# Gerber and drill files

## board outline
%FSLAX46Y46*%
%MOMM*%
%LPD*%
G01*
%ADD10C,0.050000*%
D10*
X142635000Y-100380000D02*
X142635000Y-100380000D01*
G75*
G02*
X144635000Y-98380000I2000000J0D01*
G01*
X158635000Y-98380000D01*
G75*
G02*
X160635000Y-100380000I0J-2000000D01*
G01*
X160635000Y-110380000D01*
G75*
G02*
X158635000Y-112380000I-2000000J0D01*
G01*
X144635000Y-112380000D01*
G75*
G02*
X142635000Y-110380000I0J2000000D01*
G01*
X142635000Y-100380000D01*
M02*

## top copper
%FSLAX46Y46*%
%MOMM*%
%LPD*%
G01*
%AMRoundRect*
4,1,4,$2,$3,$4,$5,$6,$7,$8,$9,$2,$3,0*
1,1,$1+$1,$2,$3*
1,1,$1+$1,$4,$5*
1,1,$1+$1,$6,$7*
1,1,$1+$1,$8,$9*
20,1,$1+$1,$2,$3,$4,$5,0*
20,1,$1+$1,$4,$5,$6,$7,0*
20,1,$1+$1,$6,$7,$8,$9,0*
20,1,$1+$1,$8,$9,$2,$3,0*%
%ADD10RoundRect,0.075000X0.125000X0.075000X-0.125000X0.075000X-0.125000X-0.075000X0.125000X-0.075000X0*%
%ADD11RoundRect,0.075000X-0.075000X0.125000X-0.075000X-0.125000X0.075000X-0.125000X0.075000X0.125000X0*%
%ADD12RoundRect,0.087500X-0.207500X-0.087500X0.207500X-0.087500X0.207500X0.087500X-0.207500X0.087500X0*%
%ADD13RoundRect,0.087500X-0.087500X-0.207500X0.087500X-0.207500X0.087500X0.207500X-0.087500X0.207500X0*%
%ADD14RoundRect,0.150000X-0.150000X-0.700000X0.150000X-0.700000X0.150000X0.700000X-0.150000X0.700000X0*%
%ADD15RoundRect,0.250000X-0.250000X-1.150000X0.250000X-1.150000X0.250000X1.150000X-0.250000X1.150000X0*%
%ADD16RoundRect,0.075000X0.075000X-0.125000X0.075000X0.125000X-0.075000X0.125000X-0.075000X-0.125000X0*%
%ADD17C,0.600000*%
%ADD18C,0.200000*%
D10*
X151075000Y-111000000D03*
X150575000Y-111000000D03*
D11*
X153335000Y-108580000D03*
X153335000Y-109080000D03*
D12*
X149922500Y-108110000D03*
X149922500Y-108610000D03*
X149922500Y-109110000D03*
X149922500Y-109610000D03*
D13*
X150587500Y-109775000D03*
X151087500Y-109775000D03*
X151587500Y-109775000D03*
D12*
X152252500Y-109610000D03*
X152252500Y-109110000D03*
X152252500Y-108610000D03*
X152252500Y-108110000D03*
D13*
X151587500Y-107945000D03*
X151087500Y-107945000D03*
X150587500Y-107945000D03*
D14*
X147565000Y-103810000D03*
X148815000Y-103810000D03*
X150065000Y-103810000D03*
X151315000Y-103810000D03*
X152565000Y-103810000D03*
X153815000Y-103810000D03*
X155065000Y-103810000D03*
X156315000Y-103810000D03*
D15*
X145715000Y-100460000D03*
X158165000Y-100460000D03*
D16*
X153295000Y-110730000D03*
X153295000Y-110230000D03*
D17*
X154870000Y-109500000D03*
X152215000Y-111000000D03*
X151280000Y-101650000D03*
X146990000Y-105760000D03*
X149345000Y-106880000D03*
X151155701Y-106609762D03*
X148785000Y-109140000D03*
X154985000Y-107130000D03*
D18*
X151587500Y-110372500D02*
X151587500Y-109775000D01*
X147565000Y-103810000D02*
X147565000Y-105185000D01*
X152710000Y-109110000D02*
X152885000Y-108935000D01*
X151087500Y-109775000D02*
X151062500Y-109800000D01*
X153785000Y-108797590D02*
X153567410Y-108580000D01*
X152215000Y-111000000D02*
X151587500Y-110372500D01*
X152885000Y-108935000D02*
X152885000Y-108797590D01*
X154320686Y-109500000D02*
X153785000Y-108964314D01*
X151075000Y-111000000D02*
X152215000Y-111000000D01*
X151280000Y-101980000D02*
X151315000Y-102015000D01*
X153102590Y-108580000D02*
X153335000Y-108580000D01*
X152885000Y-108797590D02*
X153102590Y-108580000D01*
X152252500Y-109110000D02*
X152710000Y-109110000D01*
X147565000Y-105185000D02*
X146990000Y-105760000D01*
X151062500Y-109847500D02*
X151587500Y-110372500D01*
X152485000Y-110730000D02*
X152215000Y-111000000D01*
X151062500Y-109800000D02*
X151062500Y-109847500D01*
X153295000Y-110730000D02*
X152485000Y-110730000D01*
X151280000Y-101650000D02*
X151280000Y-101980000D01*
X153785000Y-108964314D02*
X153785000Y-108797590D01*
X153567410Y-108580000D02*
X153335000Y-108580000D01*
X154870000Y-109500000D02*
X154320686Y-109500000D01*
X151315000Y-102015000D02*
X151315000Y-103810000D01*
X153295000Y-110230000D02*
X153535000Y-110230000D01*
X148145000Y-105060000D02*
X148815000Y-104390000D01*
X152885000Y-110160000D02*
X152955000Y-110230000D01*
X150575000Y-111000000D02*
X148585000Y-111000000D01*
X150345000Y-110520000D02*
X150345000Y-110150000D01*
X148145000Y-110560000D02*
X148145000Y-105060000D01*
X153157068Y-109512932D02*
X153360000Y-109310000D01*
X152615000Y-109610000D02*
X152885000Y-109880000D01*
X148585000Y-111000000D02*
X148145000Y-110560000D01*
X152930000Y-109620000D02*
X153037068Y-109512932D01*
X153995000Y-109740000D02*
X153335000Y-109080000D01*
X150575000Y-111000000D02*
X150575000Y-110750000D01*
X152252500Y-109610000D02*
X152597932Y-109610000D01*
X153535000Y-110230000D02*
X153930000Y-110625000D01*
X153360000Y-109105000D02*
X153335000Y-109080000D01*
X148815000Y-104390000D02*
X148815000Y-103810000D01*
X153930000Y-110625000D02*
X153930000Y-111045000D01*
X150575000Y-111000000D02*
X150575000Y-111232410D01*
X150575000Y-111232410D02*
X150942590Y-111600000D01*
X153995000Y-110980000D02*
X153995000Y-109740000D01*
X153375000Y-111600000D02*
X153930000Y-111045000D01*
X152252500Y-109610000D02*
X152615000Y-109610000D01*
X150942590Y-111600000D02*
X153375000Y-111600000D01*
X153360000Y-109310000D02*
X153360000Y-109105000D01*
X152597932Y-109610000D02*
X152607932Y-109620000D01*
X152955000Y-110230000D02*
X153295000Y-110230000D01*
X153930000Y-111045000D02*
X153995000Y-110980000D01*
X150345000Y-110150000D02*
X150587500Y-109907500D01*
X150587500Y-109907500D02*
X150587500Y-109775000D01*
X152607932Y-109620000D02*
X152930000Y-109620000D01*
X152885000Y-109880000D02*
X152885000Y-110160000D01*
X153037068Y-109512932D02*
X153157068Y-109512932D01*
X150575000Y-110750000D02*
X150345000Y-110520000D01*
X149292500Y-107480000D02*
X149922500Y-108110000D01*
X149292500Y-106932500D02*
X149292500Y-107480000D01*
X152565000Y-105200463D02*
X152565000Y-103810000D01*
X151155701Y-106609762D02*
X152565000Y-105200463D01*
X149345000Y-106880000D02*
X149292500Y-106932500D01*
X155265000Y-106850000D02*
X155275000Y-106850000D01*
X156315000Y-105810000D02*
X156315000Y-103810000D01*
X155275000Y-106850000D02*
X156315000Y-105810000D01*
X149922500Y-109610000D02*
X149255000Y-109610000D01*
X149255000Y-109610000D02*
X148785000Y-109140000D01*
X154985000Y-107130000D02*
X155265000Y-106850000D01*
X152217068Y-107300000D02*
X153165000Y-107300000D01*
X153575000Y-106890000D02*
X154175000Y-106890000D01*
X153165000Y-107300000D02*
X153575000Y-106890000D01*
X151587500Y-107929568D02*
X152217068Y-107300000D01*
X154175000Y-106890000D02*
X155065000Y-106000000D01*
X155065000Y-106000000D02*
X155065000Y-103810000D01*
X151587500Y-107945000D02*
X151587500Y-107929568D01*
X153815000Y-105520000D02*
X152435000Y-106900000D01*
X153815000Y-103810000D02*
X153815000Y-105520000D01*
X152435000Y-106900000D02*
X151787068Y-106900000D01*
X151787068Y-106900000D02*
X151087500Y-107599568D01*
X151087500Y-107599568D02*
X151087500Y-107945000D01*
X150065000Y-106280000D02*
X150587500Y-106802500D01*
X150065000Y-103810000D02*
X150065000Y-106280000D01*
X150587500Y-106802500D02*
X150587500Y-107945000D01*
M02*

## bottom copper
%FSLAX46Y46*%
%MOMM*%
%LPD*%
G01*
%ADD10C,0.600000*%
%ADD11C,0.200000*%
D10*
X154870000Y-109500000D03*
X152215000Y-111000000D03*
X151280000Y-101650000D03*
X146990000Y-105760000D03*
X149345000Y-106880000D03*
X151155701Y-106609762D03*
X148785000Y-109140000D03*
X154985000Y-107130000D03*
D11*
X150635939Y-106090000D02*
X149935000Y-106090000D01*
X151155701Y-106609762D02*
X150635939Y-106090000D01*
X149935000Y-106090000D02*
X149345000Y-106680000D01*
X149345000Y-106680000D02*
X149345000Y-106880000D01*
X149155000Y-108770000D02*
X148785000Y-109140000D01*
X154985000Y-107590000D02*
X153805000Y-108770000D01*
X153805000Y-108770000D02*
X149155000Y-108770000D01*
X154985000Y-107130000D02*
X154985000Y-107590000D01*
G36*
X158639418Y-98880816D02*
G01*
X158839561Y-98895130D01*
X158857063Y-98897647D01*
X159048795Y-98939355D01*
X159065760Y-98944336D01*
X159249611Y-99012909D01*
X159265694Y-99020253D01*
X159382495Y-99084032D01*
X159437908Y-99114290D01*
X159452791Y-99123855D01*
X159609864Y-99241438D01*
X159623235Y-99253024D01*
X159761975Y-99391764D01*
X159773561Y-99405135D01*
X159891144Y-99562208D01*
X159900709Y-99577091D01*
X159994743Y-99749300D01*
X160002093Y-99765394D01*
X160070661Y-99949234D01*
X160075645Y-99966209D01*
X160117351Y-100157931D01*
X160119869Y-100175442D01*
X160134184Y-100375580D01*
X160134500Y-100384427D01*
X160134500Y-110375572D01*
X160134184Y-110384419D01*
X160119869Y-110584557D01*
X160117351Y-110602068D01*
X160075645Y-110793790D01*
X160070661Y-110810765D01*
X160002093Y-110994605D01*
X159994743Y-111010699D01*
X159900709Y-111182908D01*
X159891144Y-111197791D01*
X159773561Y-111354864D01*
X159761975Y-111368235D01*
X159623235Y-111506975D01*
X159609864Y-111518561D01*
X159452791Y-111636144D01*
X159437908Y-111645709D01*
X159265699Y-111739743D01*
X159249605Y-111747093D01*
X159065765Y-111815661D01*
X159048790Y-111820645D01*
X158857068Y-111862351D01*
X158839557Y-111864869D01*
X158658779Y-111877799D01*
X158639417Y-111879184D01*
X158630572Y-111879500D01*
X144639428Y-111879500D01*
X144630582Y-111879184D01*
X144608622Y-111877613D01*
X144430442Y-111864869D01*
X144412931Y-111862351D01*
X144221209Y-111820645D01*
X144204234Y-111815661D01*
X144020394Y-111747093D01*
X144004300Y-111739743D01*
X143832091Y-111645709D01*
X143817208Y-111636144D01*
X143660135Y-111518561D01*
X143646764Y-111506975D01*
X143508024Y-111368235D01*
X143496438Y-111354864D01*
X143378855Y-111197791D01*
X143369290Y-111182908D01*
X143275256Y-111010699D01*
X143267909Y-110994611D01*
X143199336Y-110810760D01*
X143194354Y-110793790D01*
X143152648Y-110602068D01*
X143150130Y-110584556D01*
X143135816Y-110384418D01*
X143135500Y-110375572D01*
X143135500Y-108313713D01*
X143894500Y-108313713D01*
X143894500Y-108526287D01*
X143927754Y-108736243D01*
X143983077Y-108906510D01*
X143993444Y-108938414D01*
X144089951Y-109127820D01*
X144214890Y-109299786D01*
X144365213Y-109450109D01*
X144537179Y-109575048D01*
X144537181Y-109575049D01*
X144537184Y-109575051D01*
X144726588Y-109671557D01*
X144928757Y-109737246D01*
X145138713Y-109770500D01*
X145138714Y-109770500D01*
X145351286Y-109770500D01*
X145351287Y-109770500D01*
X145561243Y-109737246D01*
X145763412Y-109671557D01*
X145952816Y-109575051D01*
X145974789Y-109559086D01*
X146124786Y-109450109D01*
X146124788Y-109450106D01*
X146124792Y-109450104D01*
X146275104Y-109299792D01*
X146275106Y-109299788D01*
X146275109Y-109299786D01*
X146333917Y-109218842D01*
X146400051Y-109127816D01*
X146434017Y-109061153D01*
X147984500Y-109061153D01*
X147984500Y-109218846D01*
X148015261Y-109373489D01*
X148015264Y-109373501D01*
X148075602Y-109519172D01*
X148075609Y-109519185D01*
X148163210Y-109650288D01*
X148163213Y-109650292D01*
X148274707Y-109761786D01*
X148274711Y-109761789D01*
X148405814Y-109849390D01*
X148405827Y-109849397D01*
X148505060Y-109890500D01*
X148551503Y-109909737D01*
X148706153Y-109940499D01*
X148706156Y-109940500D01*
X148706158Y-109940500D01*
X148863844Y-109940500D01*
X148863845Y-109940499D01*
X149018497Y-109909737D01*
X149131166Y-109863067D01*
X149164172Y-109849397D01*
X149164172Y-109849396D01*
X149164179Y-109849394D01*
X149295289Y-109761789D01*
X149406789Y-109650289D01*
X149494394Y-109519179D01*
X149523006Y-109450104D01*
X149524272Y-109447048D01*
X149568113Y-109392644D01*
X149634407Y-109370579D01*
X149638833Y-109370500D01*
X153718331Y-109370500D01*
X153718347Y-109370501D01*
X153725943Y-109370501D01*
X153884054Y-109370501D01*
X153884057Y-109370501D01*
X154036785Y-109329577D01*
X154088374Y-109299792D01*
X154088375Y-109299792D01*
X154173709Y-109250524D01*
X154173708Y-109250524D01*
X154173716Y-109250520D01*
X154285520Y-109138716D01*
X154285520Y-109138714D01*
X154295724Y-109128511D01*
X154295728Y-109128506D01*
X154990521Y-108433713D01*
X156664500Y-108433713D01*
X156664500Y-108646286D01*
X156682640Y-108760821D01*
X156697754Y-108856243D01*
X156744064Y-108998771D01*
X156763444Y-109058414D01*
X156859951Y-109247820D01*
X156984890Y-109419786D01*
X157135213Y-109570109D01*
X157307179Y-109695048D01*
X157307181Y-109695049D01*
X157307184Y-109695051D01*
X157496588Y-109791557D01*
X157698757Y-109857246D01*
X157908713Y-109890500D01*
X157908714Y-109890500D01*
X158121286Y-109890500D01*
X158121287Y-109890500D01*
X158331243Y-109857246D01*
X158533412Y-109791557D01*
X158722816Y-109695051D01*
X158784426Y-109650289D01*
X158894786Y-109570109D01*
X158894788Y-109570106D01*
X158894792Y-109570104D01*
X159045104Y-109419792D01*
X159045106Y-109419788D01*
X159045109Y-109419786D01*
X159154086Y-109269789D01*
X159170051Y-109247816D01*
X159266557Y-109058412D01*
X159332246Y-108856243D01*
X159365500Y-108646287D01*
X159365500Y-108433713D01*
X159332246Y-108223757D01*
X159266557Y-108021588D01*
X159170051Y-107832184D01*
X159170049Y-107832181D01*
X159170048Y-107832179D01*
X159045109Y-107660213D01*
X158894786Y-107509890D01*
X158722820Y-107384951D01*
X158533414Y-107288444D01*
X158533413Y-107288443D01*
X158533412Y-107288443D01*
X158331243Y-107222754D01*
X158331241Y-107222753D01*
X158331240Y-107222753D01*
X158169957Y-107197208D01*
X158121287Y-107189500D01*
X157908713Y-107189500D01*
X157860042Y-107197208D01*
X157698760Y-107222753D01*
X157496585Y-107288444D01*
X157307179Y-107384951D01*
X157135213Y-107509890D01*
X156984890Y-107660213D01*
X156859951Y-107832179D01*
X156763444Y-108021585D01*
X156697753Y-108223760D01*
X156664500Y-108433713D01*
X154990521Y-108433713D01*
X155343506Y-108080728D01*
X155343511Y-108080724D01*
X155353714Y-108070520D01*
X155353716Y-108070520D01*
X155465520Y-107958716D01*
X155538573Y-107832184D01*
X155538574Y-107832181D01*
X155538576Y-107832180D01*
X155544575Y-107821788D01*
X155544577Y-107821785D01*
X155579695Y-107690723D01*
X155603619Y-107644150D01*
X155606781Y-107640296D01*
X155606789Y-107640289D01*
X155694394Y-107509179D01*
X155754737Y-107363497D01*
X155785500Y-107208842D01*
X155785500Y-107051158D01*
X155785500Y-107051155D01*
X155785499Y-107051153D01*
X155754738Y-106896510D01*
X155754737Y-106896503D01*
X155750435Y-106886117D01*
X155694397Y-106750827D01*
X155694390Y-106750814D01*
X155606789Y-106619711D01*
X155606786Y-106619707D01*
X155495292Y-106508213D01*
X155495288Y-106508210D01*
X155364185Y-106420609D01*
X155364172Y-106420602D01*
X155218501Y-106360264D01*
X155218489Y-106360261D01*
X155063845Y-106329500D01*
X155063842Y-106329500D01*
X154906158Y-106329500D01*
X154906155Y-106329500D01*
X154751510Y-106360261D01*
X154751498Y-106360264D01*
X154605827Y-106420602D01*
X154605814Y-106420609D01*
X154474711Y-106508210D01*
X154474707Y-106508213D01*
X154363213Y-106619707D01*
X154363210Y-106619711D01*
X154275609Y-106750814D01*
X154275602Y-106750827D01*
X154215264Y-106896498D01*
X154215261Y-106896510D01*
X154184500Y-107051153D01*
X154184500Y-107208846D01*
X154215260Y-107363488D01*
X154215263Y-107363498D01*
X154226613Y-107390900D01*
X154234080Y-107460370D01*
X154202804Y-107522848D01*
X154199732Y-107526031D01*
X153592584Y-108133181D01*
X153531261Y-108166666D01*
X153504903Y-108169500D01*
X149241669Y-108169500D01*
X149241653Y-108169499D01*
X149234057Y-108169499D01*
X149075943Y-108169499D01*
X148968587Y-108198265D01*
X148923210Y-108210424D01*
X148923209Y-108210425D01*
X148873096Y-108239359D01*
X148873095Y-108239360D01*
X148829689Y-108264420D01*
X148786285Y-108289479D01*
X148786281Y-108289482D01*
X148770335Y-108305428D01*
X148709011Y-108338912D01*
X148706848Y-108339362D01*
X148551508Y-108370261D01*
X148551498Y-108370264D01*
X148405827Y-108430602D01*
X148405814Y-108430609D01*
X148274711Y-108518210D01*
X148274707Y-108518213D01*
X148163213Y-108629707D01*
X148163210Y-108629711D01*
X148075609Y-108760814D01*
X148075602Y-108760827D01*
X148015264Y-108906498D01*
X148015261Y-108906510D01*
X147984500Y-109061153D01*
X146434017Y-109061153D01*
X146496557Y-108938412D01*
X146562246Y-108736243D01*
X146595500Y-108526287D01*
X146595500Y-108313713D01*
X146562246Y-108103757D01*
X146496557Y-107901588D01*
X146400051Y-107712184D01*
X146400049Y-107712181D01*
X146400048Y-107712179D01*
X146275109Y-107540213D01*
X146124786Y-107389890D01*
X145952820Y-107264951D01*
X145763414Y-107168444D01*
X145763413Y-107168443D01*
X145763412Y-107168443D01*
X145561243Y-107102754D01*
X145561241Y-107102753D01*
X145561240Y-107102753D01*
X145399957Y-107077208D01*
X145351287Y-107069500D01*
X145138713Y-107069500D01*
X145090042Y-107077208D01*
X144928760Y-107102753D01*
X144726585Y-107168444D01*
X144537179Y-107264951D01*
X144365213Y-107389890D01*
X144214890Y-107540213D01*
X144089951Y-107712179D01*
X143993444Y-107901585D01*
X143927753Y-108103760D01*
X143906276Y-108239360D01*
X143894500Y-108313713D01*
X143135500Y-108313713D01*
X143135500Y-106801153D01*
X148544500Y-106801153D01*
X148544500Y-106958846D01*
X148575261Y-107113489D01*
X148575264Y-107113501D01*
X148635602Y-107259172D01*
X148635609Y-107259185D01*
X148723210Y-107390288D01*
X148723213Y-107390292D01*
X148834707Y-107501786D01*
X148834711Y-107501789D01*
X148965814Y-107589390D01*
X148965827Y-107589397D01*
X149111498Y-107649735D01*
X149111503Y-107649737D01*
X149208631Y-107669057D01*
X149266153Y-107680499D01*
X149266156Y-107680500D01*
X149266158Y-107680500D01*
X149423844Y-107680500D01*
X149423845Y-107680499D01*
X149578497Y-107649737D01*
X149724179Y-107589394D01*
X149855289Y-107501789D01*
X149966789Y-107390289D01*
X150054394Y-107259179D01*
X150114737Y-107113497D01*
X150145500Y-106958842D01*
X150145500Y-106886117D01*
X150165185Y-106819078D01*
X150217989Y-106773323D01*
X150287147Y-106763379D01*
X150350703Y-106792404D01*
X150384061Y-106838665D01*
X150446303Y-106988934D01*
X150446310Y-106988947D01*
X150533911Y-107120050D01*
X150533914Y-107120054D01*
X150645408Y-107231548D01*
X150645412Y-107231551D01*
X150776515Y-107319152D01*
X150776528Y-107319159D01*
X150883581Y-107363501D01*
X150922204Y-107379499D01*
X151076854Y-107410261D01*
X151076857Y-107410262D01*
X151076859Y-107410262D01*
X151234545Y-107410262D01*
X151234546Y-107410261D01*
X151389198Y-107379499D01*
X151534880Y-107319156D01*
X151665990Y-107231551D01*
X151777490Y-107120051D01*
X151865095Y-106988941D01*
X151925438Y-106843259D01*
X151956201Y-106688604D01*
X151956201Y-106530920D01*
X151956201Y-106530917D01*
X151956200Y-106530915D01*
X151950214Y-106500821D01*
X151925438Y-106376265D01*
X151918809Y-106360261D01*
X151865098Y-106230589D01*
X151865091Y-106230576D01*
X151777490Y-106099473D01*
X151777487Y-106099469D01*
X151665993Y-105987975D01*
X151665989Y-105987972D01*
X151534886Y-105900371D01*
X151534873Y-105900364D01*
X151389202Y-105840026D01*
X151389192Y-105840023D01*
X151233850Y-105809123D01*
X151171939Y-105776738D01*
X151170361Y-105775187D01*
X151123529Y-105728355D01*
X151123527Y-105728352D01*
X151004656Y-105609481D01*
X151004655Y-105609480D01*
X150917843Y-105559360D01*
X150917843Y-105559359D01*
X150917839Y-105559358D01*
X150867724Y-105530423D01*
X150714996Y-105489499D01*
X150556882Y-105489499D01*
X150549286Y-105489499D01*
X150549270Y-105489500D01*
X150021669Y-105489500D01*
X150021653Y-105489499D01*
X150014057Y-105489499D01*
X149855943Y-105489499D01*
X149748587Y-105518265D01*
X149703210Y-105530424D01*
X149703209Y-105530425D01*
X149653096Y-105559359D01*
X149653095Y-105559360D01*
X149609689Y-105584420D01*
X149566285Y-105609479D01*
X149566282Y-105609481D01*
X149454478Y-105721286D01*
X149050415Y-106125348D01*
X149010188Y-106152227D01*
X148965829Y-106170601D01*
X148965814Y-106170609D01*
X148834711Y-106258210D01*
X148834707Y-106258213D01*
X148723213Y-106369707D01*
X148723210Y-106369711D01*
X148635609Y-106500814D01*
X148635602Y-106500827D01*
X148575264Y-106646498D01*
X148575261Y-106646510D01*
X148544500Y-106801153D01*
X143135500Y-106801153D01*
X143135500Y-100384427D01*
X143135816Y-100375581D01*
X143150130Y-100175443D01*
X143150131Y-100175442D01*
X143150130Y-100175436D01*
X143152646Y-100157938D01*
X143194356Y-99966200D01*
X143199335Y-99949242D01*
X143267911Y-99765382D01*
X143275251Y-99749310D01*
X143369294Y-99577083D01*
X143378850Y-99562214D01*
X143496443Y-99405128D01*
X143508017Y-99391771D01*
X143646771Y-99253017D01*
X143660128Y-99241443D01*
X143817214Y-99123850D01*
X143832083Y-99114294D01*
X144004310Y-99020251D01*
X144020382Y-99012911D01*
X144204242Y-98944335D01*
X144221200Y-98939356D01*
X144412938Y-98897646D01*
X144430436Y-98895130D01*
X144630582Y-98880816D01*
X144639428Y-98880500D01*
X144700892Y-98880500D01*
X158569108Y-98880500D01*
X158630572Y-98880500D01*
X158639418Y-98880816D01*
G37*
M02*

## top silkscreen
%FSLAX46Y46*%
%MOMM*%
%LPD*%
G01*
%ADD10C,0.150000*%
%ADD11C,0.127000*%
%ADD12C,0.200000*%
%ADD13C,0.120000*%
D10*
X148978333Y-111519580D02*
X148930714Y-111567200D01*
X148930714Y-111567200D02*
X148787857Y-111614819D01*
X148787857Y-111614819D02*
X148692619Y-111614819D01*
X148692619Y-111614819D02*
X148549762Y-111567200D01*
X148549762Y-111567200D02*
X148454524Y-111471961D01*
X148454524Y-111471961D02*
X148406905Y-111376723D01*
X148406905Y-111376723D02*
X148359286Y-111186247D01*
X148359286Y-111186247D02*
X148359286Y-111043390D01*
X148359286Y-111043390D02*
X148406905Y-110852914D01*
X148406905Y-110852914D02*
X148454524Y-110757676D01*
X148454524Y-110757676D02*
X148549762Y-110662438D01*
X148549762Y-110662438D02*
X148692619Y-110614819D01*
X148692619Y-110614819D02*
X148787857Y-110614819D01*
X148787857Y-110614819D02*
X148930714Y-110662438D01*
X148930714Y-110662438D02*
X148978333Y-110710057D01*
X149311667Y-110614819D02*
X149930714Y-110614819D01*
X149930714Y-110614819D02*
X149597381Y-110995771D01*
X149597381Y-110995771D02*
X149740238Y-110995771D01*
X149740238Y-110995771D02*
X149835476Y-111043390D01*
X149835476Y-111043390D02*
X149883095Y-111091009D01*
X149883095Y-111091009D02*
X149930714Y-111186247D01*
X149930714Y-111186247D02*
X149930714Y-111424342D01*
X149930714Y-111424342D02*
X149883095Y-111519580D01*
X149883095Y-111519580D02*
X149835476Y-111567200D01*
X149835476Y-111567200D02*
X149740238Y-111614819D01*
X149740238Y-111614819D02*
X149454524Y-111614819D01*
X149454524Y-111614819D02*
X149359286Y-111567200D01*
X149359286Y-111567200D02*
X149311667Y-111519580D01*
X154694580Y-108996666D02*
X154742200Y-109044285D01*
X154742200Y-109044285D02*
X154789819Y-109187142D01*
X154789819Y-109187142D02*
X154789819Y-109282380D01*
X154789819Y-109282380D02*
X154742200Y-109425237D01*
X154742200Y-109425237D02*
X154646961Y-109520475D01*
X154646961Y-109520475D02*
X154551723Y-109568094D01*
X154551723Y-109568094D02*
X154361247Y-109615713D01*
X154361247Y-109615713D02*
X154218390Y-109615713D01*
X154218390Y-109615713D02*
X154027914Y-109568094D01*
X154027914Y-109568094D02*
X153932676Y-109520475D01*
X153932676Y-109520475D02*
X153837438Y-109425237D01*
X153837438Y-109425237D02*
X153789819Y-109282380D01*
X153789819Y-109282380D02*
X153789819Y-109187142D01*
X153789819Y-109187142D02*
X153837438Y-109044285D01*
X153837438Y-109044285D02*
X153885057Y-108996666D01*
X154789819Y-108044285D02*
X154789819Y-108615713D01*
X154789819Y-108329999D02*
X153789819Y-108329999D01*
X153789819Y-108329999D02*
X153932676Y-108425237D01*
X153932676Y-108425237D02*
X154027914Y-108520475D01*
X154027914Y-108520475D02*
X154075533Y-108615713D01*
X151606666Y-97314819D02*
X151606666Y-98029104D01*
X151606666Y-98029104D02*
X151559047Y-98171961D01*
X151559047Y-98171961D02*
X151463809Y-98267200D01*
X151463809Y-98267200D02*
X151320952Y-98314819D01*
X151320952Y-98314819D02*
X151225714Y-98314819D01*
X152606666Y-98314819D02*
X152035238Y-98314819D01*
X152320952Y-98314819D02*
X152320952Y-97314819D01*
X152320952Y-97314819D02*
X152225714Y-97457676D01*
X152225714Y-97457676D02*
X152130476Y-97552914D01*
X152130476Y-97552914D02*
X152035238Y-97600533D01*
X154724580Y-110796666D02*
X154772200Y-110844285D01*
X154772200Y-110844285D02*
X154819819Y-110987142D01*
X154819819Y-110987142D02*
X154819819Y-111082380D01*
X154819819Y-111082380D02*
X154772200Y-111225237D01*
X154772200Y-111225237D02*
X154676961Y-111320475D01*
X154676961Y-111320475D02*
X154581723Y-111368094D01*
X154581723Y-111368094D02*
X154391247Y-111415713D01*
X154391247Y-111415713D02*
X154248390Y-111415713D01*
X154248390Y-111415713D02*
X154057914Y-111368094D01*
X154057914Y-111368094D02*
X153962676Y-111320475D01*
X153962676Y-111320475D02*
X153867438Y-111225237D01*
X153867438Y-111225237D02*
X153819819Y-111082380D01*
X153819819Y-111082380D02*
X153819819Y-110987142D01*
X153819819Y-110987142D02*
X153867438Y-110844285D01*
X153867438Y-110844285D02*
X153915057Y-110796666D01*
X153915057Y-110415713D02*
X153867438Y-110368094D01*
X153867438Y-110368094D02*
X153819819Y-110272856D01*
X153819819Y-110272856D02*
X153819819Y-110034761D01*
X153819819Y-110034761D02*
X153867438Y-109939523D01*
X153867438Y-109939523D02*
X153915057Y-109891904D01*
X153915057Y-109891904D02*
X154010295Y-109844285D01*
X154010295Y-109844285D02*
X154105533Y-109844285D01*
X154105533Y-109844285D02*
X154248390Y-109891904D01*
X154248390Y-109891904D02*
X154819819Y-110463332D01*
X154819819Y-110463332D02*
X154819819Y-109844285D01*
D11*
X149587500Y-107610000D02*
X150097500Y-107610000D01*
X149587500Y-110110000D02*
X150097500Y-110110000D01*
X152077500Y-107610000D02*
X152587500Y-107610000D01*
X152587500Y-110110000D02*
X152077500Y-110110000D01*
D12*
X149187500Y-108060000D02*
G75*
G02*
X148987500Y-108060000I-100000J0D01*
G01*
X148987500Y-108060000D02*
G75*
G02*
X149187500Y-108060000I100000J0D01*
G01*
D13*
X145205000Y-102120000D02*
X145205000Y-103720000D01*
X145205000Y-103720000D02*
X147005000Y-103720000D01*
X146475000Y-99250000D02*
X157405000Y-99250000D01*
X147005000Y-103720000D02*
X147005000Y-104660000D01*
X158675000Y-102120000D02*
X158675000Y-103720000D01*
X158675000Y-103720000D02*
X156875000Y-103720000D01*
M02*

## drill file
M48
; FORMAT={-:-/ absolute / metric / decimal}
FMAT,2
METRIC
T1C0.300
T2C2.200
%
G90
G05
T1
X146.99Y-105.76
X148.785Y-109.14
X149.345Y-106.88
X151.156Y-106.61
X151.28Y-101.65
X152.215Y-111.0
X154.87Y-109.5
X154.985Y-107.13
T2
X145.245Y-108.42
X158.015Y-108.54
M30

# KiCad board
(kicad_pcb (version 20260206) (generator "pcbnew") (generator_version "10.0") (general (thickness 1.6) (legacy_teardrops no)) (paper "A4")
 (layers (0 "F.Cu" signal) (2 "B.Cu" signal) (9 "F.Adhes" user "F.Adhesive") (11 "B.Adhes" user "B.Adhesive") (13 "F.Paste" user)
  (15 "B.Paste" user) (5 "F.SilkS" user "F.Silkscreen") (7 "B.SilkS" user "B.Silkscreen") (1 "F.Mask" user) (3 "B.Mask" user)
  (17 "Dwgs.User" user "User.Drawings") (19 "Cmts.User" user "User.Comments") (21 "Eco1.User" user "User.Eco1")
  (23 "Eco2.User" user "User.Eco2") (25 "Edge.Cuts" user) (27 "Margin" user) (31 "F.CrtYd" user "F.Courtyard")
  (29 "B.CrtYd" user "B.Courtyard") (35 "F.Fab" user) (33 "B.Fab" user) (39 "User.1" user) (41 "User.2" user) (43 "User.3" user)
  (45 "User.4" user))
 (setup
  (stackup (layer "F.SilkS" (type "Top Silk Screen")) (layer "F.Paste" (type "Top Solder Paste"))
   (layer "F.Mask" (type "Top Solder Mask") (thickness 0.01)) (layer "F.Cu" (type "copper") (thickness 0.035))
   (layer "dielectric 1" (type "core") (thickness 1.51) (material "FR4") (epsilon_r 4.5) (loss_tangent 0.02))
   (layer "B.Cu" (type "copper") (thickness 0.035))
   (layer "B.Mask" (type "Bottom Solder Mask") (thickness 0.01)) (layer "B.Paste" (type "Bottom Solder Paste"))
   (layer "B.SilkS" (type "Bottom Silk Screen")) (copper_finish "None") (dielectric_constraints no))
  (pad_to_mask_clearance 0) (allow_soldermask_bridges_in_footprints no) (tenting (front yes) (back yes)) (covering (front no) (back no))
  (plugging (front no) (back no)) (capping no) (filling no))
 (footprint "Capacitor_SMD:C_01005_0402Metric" (layer "F.Cu") (at 150.825 111 180)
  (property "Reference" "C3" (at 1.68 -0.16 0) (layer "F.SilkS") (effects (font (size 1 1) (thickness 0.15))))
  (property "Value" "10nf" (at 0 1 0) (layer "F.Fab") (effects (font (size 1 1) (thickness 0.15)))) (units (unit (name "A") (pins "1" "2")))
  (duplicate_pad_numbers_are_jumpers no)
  (pad "" smd roundrect (at -0.275 0 180) (size 0.27 0.27) (layers "F.Paste") (roundrect_rratio 0.25))
  (pad "" smd roundrect (at 0.275 0 180) (size 0.27 0.27) (layers "F.Paste") (roundrect_rratio 0.25))
  (pad "1" smd roundrect (at -0.25 0 180) (size 0.4 0.3) (layers "F.Cu" "F.Mask") (roundrect_rratio 0.25) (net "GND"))
  (pad "2" smd roundrect (at 0.25 0 180) (size 0.4 0.3) (layers "F.Cu" "F.Mask") (roundrect_rratio 0.25) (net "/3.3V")))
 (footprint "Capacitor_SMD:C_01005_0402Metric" (layer "F.Cu") (at 153.335 108.83 -90)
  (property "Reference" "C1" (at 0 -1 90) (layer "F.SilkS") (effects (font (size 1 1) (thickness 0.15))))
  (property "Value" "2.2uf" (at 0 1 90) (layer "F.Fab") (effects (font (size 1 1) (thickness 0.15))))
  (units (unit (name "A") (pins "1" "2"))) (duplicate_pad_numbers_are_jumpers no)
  (pad "" smd roundrect (at -0.275 0 270) (size 0.27 0.27) (layers "F.Paste") (roundrect_rratio 0.25))
  (pad "" smd roundrect (at 0.275 0 270) (size 0.27 0.27) (layers "F.Paste") (roundrect_rratio 0.25))
  (pad "1" smd roundrect (at -0.25 0 270) (size 0.4 0.3) (layers "F.Cu" "F.Mask") (roundrect_rratio 0.25) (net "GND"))
  (pad "2" smd roundrect (at 0.25 0 270) (size 0.4 0.3) (layers "F.Cu" "F.Mask") (roundrect_rratio 0.25) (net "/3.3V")))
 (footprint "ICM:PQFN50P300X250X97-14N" (layer "F.Cu") (at 151.0875 108.86)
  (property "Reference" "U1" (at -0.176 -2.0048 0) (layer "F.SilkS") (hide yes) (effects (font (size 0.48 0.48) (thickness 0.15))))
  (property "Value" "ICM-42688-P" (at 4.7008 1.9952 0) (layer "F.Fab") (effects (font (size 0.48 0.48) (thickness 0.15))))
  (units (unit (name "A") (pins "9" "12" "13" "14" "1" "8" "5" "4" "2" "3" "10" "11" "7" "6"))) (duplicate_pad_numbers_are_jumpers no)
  (fp_line (start -1.5 -1.25) (end -0.99 -1.25) (stroke (width 0.127) (type solid)) (layer "F.SilkS"))
  (fp_line (start -1.5 1.25) (end -0.99 1.25) (stroke (width 0.127) (type solid)) (layer "F.SilkS"))
  (fp_line (start 0.99 -1.25) (end 1.5 -1.25) (stroke (width 0.127) (type solid)) (layer "F.SilkS"))
  (fp_line (start 1.5 1.25) (end 0.99 1.25) (stroke (width 0.127) (type solid)) (layer "F.SilkS"))
  (fp_circle (center -2 -0.8) (end -1.9 -0.8) (stroke (width 0.2) (type solid)) (fill no) (layer "F.SilkS"))
  (pad "1" smd roundrect (at -1.165 -0.75) (size 0.59 0.35) (layers "F.Cu" "F.Paste") (roundrect_rratio 0.25) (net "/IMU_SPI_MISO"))
  (pad "2" smd roundrect (at -1.165 -0.25) (size 0.59 0.35) (layers "F.Cu" "F.Paste") (roundrect_rratio 0.25)
   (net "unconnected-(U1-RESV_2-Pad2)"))
  (pad "3" smd roundrect (at -1.165 0.25) (size 0.59 0.35) (layers "F.Cu" "F.Paste") (roundrect_rratio 0.25)
   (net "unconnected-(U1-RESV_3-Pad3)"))
  (pad "4" smd roundrect (at -1.165 0.75) (size 0.59 0.35) (layers "F.Cu" "F.Paste") (roundrect_rratio 0.25) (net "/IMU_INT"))
  (pad "5" smd roundrect (at -0.5 0.915) (size 0.35 0.59) (layers "F.Cu" "F.Paste") (roundrect_rratio 0.25) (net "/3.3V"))
  (pad "6" smd roundrect (at 0 0.915) (size 0.35 0.59) (layers "F.Cu" "F.Paste") (roundrect_rratio 0.25) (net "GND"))
  (pad "7" smd roundrect (at 0.5 0.915) (size 0.35 0.59) (layers "F.Cu" "F.Paste") (roundrect_rratio 0.25) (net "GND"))
  (pad "8" smd roundrect (at 1.165 0.75) (size 0.59 0.35) (layers "F.Cu" "F.Paste") (roundrect_rratio 0.25) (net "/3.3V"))
  (pad "9" smd roundrect (at 1.165 0.25) (size 0.59 0.35) (layers "F.Cu" "F.Paste") (roundrect_rratio 0.25) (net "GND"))
  (pad "10" smd roundrect (at 1.165 -0.25) (size 0.59 0.35) (layers "F.Cu" "F.Paste") (roundrect_rratio 0.25)
   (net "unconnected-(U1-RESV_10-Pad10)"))
  (pad "11" smd roundrect (at 1.165 -0.75) (size 0.59 0.35) (layers "F.Cu" "F.Paste") (roundrect_rratio 0.25)
   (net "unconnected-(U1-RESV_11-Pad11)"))
  (pad "12" smd roundrect (at 0.5 -0.915) (size 0.35 0.59) (layers "F.Cu" "F.Paste") (roundrect_rratio 0.25) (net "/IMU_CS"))
  (pad "13" smd roundrect (at 0 -0.915) (size 0.35 0.59) (layers "F.Cu" "F.Paste") (roundrect_rratio 0.25) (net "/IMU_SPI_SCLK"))
  (pad "14" smd roundrect (at -0.5 -0.915) (size 0.35 0.59) (layers "F.Cu" "F.Paste") (roundrect_rratio 0.25) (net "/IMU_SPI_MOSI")))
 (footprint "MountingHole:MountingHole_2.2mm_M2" (layer "F.Cu") (at 158.015 108.54)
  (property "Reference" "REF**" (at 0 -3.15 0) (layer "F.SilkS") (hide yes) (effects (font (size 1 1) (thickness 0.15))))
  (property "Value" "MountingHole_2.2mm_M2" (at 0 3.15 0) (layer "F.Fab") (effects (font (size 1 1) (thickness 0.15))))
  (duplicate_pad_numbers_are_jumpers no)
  (pad "" np_thru_hole circle (at 0 0) (size 2.2 2.2) (drill 2.2) (layers "*.Cu" "*.Mask")))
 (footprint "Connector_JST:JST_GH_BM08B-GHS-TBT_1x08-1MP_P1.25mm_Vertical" (layer "F.Cu") (at 151.94 101.86)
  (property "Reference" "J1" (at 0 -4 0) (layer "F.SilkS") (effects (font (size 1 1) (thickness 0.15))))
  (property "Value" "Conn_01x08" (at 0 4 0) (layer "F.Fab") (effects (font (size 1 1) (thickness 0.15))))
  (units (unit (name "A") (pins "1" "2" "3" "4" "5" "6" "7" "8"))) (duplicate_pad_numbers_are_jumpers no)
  (fp_line (start -6.735 0.26) (end -6.735 1.86) (stroke (width 0.12) (type solid)) (layer "F.SilkS"))
  (fp_line (start -6.735 1.86) (end -4.935 1.86) (stroke (width 0.12) (type solid)) (layer "F.SilkS"))
  (fp_line (start -5.465 -2.61) (end 5.465 -2.61) (stroke (width 0.12) (type solid)) (layer "F.SilkS"))
  (fp_line (start -4.935 1.86) (end -4.935 2.8) (stroke (width 0.12) (type solid)) (layer "F.SilkS"))
  (fp_line (start 6.735 0.26) (end 6.735 1.86) (stroke (width 0.12) (type solid)) (layer "F.SilkS"))
  (fp_line (start 6.735 1.86) (end 4.935 1.86) (stroke (width 0.12) (type solid)) (layer "F.SilkS"))
  (pad "1" smd roundrect (at -4.375 1.95) (size 0.6 1.7) (layers "F.Cu" "F.Mask" "F.Paste") (roundrect_rratio 0.25) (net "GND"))
  (pad "2" smd roundrect (at -3.125 1.95) (size 0.6 1.7) (layers "F.Cu" "F.Mask" "F.Paste") (roundrect_rratio 0.25) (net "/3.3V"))
  (pad "3" smd roundrect (at -1.875 1.95) (size 0.6 1.7) (layers "F.Cu" "F.Mask" "F.Paste") (roundrect_rratio 0.25) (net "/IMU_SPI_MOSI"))
  (pad "4" smd roundrect (at -0.625 1.95) (size 0.6 1.7) (layers "F.Cu" "F.Mask" "F.Paste") (roundrect_rratio 0.25) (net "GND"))
  (pad "5" smd roundrect (at 0.625 1.95) (size 0.6 1.7) (layers "F.Cu" "F.Mask" "F.Paste") (roundrect_rratio 0.25) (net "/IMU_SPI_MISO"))
  (pad "6" smd roundrect (at 1.875 1.95) (size 0.6 1.7) (layers "F.Cu" "F.Mask" "F.Paste") (roundrect_rratio 0.25) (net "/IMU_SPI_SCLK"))
  (pad "7" smd roundrect (at 3.125 1.95) (size 0.6 1.7) (layers "F.Cu" "F.Mask" "F.Paste") (roundrect_rratio 0.25) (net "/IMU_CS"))
  (pad "8" smd roundrect (at 4.375 1.95) (size 0.6 1.7) (layers "F.Cu" "F.Mask" "F.Paste") (roundrect_rratio 0.25) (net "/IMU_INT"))
  (pad "MP" smd roundrect (at -6.225 -1.4) (size 1 2.8) (layers "F.Cu" "F.Mask" "F.Paste") (roundrect_rratio 0.25))
  (pad "MP" smd roundrect (at 6.225 -1.4) (size 1 2.8) (layers "F.Cu" "F.Mask" "F.Paste") (roundrect_rratio 0.25)))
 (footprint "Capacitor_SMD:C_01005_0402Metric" (layer "F.Cu") (at 153.295 110.48 90)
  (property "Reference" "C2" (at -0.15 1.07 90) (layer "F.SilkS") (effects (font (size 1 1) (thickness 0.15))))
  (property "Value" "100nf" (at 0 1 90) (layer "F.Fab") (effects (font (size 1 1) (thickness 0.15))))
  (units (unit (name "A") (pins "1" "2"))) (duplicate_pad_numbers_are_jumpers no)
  (pad "" smd roundrect (at -0.275 0 90) (size 0.27 0.27) (layers "F.Paste") (roundrect_rratio 0.25))
  (pad "" smd roundrect (at 0.275 0 90) (size 0.27 0.27) (layers "F.Paste") (roundrect_rratio 0.25))
  (pad "1" smd roundrect (at -0.25 0 90) (size 0.4 0.3) (layers "F.Cu" "F.Mask") (roundrect_rratio 0.25) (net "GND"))
  (pad "2" smd roundrect (at 0.25 0 90) (size 0.4 0.3) (layers "F.Cu" "F.Mask") (roundrect_rratio 0.25) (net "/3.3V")))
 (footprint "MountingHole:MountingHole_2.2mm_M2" (layer "F.Cu") (at 145.245 108.42)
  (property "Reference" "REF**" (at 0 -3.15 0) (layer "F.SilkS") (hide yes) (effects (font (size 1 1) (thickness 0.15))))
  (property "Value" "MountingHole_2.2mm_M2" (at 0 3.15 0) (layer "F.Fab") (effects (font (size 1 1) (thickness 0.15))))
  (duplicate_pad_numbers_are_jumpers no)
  (pad "" np_thru_hole circle (at 0 0) (size 2.2 2.2) (drill 2.2) (layers "*.Cu" "*.Mask")))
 (gr_rect (start 142.635 98.38) (end 160.635 112.38) (radius 2) (stroke (width 0.05) (type solid)) (fill no) (layer "Edge.Cuts"))
 (segment (start 151.5875 110.3725) (end 151.5875 109.775) (width 0.2) (layer "F.Cu") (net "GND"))
 (segment (start 147.565 103.81) (end 147.565 105.185) (width 0.2) (layer "F.Cu") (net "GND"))
 (segment (start 152.71 109.11) (end 152.885 108.935) (width 0.2) (layer "F.Cu") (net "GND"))
 (segment (start 151.0875 109.775) (end 151.0625 109.8) (width 0.2) (layer "F.Cu") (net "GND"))
 (segment (start 153.785 108.79759) (end 153.56741 108.58) (width 0.2) (layer "F.Cu") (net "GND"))
 (segment (start 152.215 111) (end 151.5875 110.3725) (width 0.2) (layer "F.Cu") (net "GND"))
 (segment (start 152.885 108.935) (end 152.885 108.79759) (width 0.2) (layer "F.Cu") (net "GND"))
 (segment (start 154.320686 109.5) (end 153.785 108.964314) (width 0.2) (layer "F.Cu") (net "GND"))
 (segment (start 151.075 111) (end 152.215 111) (width 0.2) (layer "F.Cu") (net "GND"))
 (segment (start 151.28 101.98) (end 151.315 102.015) (width 0.2) (layer "F.Cu") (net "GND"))
 (segment (start 153.10259 108.58) (end 153.335 108.58) (width 0.2) (layer "F.Cu") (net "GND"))
 (segment (start 152.885 108.79759) (end 153.10259 108.58) (width 0.2) (layer "F.Cu") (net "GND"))
 (segment (start 152.2525 109.11) (end 152.71 109.11) (width 0.2) (layer "F.Cu") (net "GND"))
 (segment (start 147.565 105.185) (end 146.99 105.76) (width 0.2) (layer "F.Cu") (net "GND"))
 (segment (start 151.0625 109.8475) (end 151.5875 110.3725) (width 0.2) (layer "F.Cu") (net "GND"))
 (segment (start 152.485 110.73) (end 152.215 111) (width 0.2) (layer "F.Cu") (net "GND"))
 (segment (start 151.0625 109.8) (end 151.0625 109.8475) (width 0.2) (layer "F.Cu") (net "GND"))
 (segment (start 153.295 110.73) (end 152.485 110.73) (width 0.2) (layer "F.Cu") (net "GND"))
 (segment (start 151.28 101.65) (end 151.28 101.98) (width 0.2) (layer "F.Cu") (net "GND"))
 (segment (start 153.785 108.964314) (end 153.785 108.79759) (width 0.2) (layer "F.Cu") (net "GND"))
 (segment (start 153.56741 108.58) (end 153.335 108.58) (width 0.2) (layer "F.Cu") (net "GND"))
 (segment (start 154.87 109.5) (end 154.320686 109.5) (width 0.2) (layer "F.Cu") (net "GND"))
 (segment (start 151.315 102.015) (end 151.315 103.81) (width 0.2) (layer "F.Cu") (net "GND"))
 (via (at 154.87 109.5) (size 0.6) (drill 0.3) (layers "F.Cu" "B.Cu") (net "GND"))
 (via (at 152.215 111) (size 0.6) (drill 0.3) (layers "F.Cu" "B.Cu") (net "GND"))
 (via (at 151.28 101.65) (size 0.6) (drill 0.3) (layers "F.Cu" "B.Cu") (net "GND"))
 (via (at 146.99 105.76) (size 0.6) (drill 0.3) (layers "F.Cu" "B.Cu") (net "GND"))
 (segment (start 153.295 110.23) (end 153.535 110.23) (width 0.2) (layer "F.Cu") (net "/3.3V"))
 (segment (start 148.145 105.06) (end 148.815 104.39) (width 0.2) (layer "F.Cu") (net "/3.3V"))
 (segment (start 152.885 110.16) (end 152.955 110.23) (width 0.2) (layer "F.Cu") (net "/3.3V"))
 (segment (start 150.575 111) (end 148.585 111) (width 0.2) (layer "F.Cu") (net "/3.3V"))
 (segment (start 150.345 110.52) (end 150.345 110.15) (width 0.2) (layer "F.Cu") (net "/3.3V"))
 (segment (start 148.145 110.56) (end 148.145 105.06) (width 0.2) (layer "F.Cu") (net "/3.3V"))
 (segment (start 153.157068 109.512932) (end 153.36 109.31) (width 0.2) (layer "F.Cu") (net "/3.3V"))
 (segment (start 152.615 109.61) (end 152.885 109.88) (width 0.2) (layer "F.Cu") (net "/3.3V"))
 (segment (start 148.585 111) (end 148.145 110.56) (width 0.2) (layer "F.Cu") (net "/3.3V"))
 (segment (start 152.93 109.62) (end 153.037068 109.512932) (width 0.2) (layer "F.Cu") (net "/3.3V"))
 (segment (start 153.995 109.74) (end 153.335 109.08) (width 0.2) (layer "F.Cu") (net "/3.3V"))
 (segment (start 150.575 111) (end 150.575 110.75) (width 0.2) (layer "F.Cu") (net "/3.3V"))
 (segment (start 152.2525 109.61) (end 152.597932 109.61) (width 0.2) (layer "F.Cu") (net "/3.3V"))
 (segment (start 153.535 110.23) (end 153.93 110.625) (width 0.2) (layer "F.Cu") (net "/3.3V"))
 (segment (start 153.36 109.105) (end 153.335 109.08) (width 0.2) (layer "F.Cu") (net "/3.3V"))
 (segment (start 148.815 104.39) (end 148.815 103.81) (width 0.2) (layer "F.Cu") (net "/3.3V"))
 (segment (start 153.93 110.625) (end 153.93 111.045) (width 0.2) (layer "F.Cu") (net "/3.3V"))
 (segment (start 150.575 111) (end 150.575 111.23241) (width 0.2) (layer "F.Cu") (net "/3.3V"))
 (segment (start 150.575 111.23241) (end 150.94259 111.6) (width 0.2) (layer "F.Cu") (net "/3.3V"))
 (segment (start 153.995 110.98) (end 153.995 109.74) (width 0.2) (layer "F.Cu") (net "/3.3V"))
 (segment (start 153.375 111.6) (end 153.93 111.045) (width 0.2) (layer "F.Cu") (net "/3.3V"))
 (segment (start 152.2525 109.61) (end 152.615 109.61) (width 0.2) (layer "F.Cu") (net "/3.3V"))
 (segment (start 150.94259 111.6) (end 153.375 111.6) (width 0.2) (layer "F.Cu") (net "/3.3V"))
 (segment (start 153.36 109.31) (end 153.36 109.105) (width 0.2) (layer "F.Cu") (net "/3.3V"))
 (segment (start 152.597932 109.61) (end 152.607932 109.62) (width 0.2) (layer "F.Cu") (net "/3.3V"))
 (segment (start 152.955 110.23) (end 153.295 110.23) (width 0.2) (layer "F.Cu") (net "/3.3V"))
 (segment (start 153.93 111.045) (end 153.995 110.98) (width 0.2) (layer "F.Cu") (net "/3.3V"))
 (segment (start 150.345 110.15) (end 150.5875 109.9075) (width 0.2) (layer "F.Cu") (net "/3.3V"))
 (segment (start 150.5875 109.9075) (end 150.5875 109.775) (width 0.2) (layer "F.Cu") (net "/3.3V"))
 (segment (start 152.607932 109.62) (end 152.93 109.62) (width 0.2) (layer "F.Cu") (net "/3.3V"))
 (segment (start 152.885 109.88) (end 152.885 110.16) (width 0.2) (layer "F.Cu") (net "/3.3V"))
 (segment (start 153.037068 109.512932) (end 153.157068 109.512932) (width 0.2) (layer "F.Cu") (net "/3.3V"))
 (segment (start 150.575 110.75) (end 150.345 110.52) (width 0.2) (layer "F.Cu") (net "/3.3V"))
 (segment (start 149.2925 107.48) (end 149.9225 108.11) (width 0.2) (layer "F.Cu") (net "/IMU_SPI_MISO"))
 (segment (start 149.2925 106.9325) (end 149.2925 107.48) (width 0.2) (layer "F.Cu") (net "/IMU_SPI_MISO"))
 (segment (start 152.565 105.200463) (end 152.565 103.81) (width 0.2) (layer "F.Cu") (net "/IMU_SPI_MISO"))
 (segment (start 151.155701 106.609762) (end 152.565 105.200463) (width 0.2) (layer "F.Cu") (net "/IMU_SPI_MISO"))
 (segment (start 149.345 106.88) (end 149.2925 106.9325) (width 0.2) (layer "F.Cu") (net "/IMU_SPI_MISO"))
 (via (at 149.345 106.88) (size 0.6) (drill 0.3) (layers "F.Cu" "B.Cu") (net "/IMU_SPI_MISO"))
 (via (at 151.155701 106.609762) (size 0.6) (drill 0.3) (layers "F.Cu" "B.Cu") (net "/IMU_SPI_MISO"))
 (segment (start 150.635939 106.09) (end 149.935 106.09) (width 0.2) (layer "B.Cu") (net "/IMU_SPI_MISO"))
 (segment (start 151.155701 106.609762) (end 150.635939 106.09) (width 0.2) (layer "B.Cu") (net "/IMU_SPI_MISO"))
 (segment (start 149.935 106.09) (end 149.345 106.68) (width 0.2) (layer "B.Cu") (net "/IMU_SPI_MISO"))
 (segment (start 149.345 106.68) (end 149.345 106.88) (width 0.2) (layer "B.Cu") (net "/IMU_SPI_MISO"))
 (segment (start 155.265 106.85) (end 155.275 106.85) (width 0.2) (layer "F.Cu") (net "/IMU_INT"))
 (segment (start 156.315 105.81) (end 156.315 103.81) (width 0.2) (layer "F.Cu") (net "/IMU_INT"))
 (segment (start 155.275 106.85) (end 156.315 105.81) (width 0.2) (layer "F.Cu") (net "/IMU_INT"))
 (segment (start 149.9225 109.61) (end 149.255 109.61) (width 0.2) (layer "F.Cu") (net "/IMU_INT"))
 (segment (start 149.255 109.61) (end 148.785 109.14) (width 0.2) (layer "F.Cu") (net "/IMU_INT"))
 (segment (start 154.985 107.13) (end 155.265 106.85) (width 0.2) (layer "F.Cu") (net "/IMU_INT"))
 (via (at 148.785 109.14) (size 0.6) (drill 0.3) (layers "F.Cu" "B.Cu") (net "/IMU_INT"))
 (via (at 154.985 107.13) (size 0.6) (drill 0.3) (layers "F.Cu" "B.Cu") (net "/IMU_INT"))
 (segment (start 149.155 108.77) (end 148.785 109.14) (width 0.2) (layer "B.Cu") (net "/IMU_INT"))
 (segment (start 154.985 107.59) (end 153.805 108.77) (width 0.2) (layer "B.Cu") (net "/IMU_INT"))
 (segment (start 153.805 108.77) (end 149.155 108.77) (width 0.2) (layer "B.Cu") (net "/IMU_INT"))
 (segment (start 154.985 107.13) (end 154.985 107.59) (width 0.2) (layer "B.Cu") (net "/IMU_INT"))
 (segment (start 152.217068 107.3) (end 153.165 107.3) (width 0.2) (layer "F.Cu") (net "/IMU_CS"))
 (segment (start 153.575 106.89) (end 154.175 106.89) (width 0.2) (layer "F.Cu") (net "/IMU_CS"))
 (segment (start 153.165 107.3) (end 153.575 106.89) (width 0.2) (layer "F.Cu") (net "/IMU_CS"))
 (segment (start 151.5875 107.929568) (end 152.217068 107.3) (width 0.2) (layer "F.Cu") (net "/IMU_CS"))
 (segment (start 154.175 106.89) (end 155.065 106) (width 0.2) (layer "F.Cu") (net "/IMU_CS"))
 (segment (start 155.065 106) (end 155.065 103.81) (width 0.2) (layer "F.Cu") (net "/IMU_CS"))
 (segment (start 151.5875 107.945) (end 151.5875 107.929568) (width 0.2) (layer "F.Cu") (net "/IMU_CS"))
 (segment (start 153.815 105.52) (end 152.435 106.9) (width 0.2) (layer "F.Cu") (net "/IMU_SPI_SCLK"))
 (segment (start 153.815 103.81) (end 153.815 105.52) (width 0.2) (layer "F.Cu") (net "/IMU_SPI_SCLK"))
 (segment (start 152.435 106.9) (end 151.787068 106.9) (width 0.2) (layer "F.Cu") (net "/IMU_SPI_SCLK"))
 (segment (start 151.787068 106.9) (end 151.0875 107.599568) (width 0.2) (layer "F.Cu") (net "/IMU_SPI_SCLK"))
 (segment (start 151.0875 107.599568) (end 151.0875 107.945) (width 0.2) (layer "F.Cu") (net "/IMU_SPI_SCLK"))
 (segment (start 150.065 106.28) (end 150.5875 106.8025) (width 0.2) (layer "F.Cu") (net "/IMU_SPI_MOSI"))
 (segment (start 150.065 103.81) (end 150.065 106.28) (width 0.2) (layer "F.Cu") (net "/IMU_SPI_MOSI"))
 (segment (start 150.5875 106.8025) (end 150.5875 107.945) (width 0.2) (layer "F.Cu") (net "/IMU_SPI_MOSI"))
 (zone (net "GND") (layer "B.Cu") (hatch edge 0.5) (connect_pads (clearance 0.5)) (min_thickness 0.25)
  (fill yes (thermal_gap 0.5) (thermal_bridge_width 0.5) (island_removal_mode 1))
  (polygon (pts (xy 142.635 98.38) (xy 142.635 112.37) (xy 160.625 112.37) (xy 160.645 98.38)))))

